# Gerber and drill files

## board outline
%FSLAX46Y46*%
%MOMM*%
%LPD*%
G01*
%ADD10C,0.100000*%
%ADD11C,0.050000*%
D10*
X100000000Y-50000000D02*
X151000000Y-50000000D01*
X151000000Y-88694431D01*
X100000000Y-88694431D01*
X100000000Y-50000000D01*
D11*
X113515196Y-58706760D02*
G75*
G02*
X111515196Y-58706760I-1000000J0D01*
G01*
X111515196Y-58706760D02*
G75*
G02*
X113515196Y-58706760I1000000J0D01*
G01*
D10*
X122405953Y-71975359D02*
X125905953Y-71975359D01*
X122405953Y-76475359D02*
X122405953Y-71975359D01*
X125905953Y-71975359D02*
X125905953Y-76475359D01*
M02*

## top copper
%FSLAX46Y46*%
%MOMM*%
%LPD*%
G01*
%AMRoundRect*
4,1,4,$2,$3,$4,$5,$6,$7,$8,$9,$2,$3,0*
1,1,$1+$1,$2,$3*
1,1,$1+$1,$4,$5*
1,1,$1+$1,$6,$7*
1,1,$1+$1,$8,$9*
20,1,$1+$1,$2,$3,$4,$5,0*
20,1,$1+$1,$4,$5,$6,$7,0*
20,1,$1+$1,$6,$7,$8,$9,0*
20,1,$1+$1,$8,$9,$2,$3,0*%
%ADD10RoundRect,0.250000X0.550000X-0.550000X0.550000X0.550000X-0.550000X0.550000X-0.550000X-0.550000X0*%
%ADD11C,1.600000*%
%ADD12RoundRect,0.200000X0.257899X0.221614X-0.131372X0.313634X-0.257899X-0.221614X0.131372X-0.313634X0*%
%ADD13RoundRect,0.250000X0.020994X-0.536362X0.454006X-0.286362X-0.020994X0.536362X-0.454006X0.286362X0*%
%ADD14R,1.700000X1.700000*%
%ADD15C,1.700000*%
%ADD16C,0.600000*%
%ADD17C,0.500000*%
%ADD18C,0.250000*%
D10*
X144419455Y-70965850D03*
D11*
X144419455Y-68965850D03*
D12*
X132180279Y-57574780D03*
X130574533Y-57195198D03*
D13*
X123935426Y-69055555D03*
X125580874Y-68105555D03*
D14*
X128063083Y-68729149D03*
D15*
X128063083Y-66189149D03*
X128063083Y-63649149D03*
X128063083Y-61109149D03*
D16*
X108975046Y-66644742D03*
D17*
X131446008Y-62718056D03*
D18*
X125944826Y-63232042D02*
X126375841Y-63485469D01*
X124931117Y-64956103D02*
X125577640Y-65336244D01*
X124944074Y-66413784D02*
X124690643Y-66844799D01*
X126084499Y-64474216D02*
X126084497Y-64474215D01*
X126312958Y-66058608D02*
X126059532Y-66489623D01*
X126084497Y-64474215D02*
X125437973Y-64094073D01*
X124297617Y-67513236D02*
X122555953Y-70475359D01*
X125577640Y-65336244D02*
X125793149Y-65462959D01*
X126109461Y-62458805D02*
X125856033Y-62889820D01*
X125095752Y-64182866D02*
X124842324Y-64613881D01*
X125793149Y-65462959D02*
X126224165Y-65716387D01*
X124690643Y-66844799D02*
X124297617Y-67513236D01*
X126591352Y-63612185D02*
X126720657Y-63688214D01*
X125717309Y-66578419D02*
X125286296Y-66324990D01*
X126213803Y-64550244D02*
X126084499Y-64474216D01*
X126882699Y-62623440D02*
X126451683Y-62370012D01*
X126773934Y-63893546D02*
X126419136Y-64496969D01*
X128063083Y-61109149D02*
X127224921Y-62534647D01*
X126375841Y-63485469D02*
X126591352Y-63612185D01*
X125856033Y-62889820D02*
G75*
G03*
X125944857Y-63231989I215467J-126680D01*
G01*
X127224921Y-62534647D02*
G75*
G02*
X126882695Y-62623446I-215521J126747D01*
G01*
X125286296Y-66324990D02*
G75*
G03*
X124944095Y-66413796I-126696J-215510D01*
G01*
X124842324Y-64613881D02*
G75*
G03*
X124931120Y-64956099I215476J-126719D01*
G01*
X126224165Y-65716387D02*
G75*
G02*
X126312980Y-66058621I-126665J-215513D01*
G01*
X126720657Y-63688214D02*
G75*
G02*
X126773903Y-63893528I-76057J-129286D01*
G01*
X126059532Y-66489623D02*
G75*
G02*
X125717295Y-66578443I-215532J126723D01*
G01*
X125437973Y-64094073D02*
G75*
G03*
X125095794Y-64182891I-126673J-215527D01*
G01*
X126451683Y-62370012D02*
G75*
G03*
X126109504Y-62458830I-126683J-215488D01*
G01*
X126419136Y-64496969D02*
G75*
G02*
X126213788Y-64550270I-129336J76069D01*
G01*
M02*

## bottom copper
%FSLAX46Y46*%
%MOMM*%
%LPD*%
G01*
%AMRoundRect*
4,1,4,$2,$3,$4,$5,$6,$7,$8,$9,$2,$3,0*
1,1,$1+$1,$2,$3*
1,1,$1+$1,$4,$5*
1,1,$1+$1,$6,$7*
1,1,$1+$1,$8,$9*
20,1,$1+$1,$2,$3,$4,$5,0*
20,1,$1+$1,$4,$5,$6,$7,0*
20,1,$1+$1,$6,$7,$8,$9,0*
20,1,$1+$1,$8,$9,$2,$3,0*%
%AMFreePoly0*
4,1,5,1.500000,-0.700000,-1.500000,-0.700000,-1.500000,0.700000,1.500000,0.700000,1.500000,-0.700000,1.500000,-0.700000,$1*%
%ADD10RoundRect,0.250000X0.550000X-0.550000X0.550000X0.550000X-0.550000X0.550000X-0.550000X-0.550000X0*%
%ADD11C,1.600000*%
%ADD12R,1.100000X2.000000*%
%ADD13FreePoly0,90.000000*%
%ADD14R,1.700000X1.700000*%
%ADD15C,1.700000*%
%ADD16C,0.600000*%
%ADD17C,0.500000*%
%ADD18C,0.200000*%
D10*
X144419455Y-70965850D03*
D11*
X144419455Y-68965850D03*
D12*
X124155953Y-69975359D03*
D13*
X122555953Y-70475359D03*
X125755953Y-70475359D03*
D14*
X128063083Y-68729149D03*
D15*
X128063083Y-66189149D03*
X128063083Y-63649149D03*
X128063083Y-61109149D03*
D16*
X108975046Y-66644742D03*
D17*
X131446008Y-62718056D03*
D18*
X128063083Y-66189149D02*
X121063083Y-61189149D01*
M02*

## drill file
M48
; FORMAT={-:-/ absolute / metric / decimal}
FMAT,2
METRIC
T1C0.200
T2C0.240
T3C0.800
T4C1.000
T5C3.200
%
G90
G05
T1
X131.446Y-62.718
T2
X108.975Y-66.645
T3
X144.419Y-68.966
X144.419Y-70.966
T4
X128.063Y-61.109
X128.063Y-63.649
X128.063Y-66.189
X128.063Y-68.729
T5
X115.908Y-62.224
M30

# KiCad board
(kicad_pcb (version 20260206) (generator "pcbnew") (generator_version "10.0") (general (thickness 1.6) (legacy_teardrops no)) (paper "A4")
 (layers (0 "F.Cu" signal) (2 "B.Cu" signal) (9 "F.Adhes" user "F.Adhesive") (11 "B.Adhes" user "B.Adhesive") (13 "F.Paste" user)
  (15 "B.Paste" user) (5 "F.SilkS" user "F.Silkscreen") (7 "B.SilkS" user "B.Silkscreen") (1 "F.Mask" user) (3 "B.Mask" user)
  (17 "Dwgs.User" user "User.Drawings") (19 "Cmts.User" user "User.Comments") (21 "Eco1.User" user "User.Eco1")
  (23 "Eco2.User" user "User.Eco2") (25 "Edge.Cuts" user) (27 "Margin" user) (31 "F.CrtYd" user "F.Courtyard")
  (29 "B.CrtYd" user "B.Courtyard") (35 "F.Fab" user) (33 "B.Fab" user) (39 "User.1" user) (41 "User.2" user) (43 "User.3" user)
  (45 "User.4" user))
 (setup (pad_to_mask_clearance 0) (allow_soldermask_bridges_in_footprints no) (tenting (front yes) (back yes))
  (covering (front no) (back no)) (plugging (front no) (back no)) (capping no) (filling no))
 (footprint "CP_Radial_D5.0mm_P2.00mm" (layer "F.Cu") (at 144.419455 70.96585 90)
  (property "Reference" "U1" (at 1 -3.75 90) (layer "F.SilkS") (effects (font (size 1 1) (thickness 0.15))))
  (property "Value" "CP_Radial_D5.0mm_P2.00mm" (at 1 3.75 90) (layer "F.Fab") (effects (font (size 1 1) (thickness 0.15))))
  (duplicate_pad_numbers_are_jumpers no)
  (pad "1" thru_hole roundrect (at 0 0 90) (size 1.6 1.6) (drill 0.8) (layers "*.Cu" "*.Mask") (remove_unused_layers no)
   (roundrect_rratio 0.15625) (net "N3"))
  (pad "2" thru_hole circle (at 2 0 90) (size 1.6 1.6) (drill 0.8) (layers "*.Cu" "*.Mask") (remove_unused_layers no) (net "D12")))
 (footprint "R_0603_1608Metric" (layer "F.Cu") (at 131.377406 57.384989 166.7)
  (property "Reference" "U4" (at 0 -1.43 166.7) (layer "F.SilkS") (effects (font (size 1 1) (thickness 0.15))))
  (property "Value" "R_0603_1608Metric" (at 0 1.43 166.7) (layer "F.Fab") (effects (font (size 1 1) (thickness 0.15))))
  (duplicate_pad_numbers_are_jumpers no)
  (pad "1" smd roundrect (at -0.825 0 166.7) (size 0.8 0.95) (layers "F.Cu" "F.Mask" "F.Paste") (roundrect_rratio 0.25) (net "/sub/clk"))
  (pad "2" smd roundrect (at 0.825 0 166.7) (size 0.8 0.95) (layers "F.Cu" "F.Mask" "F.Paste") (roundrect_rratio 0.25) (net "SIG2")))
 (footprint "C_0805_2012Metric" (layer "F.Cu") (at 124.75815 68.580555 30)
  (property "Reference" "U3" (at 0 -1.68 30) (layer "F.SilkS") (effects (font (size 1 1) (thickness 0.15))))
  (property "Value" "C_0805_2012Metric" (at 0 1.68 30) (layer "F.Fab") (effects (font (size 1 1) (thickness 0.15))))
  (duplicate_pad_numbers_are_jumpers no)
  (pad "1" smd roundrect (at -0.95 0 30) (size 1 1.45) (layers "F.Cu" "F.Mask" "F.Paste") (roundrect_rratio 0.25) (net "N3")
   (clearance 0.35))
  (pad "2" smd roundrect (at 0.95 0 30) (size 1 1.45) (layers "F.Cu" "F.Mask" "F.Paste") (roundrect_rratio 0.25)))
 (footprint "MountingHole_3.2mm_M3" (layer "F.Cu") (at 115.908484 62.224067 45)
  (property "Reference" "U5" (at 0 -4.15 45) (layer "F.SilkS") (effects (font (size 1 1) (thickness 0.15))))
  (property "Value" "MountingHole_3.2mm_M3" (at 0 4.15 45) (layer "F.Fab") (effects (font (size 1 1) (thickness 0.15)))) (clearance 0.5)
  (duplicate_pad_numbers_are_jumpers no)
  (pad "" np_thru_hole circle (at 0 0 45) (size 3.2 3.2) (drill 3.2) (layers "*.Cu" "*.Mask")))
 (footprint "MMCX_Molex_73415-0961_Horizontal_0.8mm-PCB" (layer "B.Cu") (at 124.155953 72.725359 90)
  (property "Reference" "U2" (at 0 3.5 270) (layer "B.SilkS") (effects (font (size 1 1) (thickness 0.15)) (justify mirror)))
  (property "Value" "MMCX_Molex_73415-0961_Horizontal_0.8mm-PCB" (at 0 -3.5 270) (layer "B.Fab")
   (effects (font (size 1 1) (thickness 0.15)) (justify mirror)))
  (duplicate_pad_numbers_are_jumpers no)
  (fp_line (start 0.75 -1.75) (end 0.75 1.75) (stroke (width 0.1) (type solid)) (layer "Edge.Cuts"))
  (fp_line (start -3.75 -1.75) (end 0.75 -1.75) (stroke (width 0.1) (type solid)) (layer "Edge.Cuts"))
  (fp_line (start 0.75 1.75) (end -3.75 1.75) (stroke (width 0.1) (type solid)) (layer "Edge.Cuts"))
  (pad "1" smd rect (at 2.75 0 90) (size 2 1.1) (layers "B.Cu" "B.Mask" "B.Paste") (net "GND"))
  (pad "2" smd custom (at 2.25 -1.6 90) (size 3 1.4) (layers "B.Cu" "B.Mask" "B.Paste") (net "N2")
   (options (clearance outline) (anchor rect)) (primitives))
  (pad "2" smd custom (at 2.25 1.6 90) (size 3 1.4) (layers "B.Cu" "B.Mask" "B.Paste") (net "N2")
   (options (clearance outline) (anchor rect)) (primitives)))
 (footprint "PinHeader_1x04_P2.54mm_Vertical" (layer "B.Cu") (at 128.063083 68.729149)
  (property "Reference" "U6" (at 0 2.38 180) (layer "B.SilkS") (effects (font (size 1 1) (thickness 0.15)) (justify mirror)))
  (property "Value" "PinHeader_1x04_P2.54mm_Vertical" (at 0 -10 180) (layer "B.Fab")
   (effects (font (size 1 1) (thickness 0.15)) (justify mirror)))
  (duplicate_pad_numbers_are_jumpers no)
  (pad "1" thru_hole rect (at 0 0) (size 1.7 1.7) (drill 1) (layers "*.Cu" "*.Mask") (remove_unused_layers no) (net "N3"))
  (pad "2" thru_hole circle (at 0 -2.54) (size 1.7 1.7) (drill 1) (layers "*.Cu" "*.Mask") (remove_unused_layers no) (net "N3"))
  (pad "3" thru_hole circle (at 0 -5.08) (size 1.7 1.7) (drill 1) (layers "*.Cu" "*.Mask") (remove_unused_layers no) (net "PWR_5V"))
  (pad "4" thru_hole circle (at 0 -7.62) (size 1.7 1.7) (drill 1) (layers "*.Cu" "*.Mask") (remove_unused_layers no)))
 (gr_rect (start 100 50) (end 151 88.694431) (stroke (width 0.1) (type default)) (fill no) (layer "Edge.Cuts"))
 (gr_circle (center 112.515196 58.70676) (end 113.515196 58.70676) (stroke (width 0.05) (type default)) (fill no) (layer "Edge.Cuts"))
 (segment (start 125.944826 63.232042) (end 126.375841 63.485469) (width 0.25) (layer "F.Cu") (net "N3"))
 (segment (start 124.931117 64.956103) (end 125.57764 65.336244) (width 0.25) (layer "F.Cu") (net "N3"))
 (segment (start 124.944074 66.413784) (end 124.690643 66.844799) (width 0.25) (layer "F.Cu") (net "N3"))
 (segment (start 126.084499 64.474216) (end 126.084497 64.474215) (width 0.25) (layer "F.Cu") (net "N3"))
 (segment (start 126.312958 66.058608) (end 126.059532 66.489623) (width 0.25) (layer "F.Cu") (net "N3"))
 (segment (start 126.084497 64.474215) (end 125.437973 64.094073) (width 0.25) (layer "F.Cu") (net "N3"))
 (segment (start 124.297617 67.513236) (end 122.555953 70.475359) (width 0.25) (layer "F.Cu") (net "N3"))
 (segment (start 125.57764 65.336244) (end 125.793149 65.462959) (width 0.25) (layer "F.Cu") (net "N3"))
 (segment (start 126.109461 62.458805) (end 125.856033 62.88982) (width 0.25) (layer "F.Cu") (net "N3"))
 (segment (start 125.095752 64.182866) (end 124.842324 64.613881) (width 0.25) (layer "F.Cu") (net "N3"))
 (segment (start 125.793149 65.462959) (end 126.224165 65.716387) (width 0.25) (layer "F.Cu") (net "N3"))
 (segment (start 124.690643 66.844799) (end 124.297617 67.513236) (width 0.25) (layer "F.Cu") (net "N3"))
 (segment (start 126.591352 63.612185) (end 126.720657 63.688214) (width 0.25) (layer "F.Cu") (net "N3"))
 (segment (start 125.717309 66.578419) (end 125.286296 66.32499) (width 0.25) (layer "F.Cu") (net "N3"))
 (segment (start 126.213803 64.550244) (end 126.084499 64.474216) (width 0.25) (layer "F.Cu") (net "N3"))
 (segment (start 126.882699 62.62344) (end 126.451683 62.370012) (width 0.25) (layer "F.Cu") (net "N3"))
 (segment (start 126.773934 63.893546) (end 126.419136 64.496969) (width 0.25) (layer "F.Cu") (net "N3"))
 (segment (start 128.063083 61.109149) (end 127.224921 62.534647) (width 0.25) (layer "F.Cu") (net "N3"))
 (segment (start 126.375841 63.485469) (end 126.591352 63.612185) (width 0.25) (layer "F.Cu") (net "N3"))
 (arc (start 125.856033 62.88982) (mid 125.829553 63.07932) (end 125.944826 63.232042) (width 0.25) (layer "F.Cu") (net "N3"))
 (arc (start 127.224921 62.534647) (mid 127.072199 62.64992) (end 126.882699 62.62344) (width 0.25) (layer "F.Cu") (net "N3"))
 (arc (start 125.286296 66.32499) (mid 125.096795 66.298511) (end 124.944074 66.413784) (width 0.25) (layer "F.Cu") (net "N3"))
 (arc (start 124.842324 64.613881) (mid 124.815844 64.803381) (end 124.931117 64.956103) (width 0.25) (layer "F.Cu") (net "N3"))
 (arc (start 126.224165 65.716387) (mid 126.339439 65.869107) (end 126.312958 66.058608) (width 0.25) (layer "F.Cu") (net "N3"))
 (arc (start 126.720657 63.688214) (mid 126.789821 63.779846) (end 126.773934 63.893546) (width 0.25) (layer "F.Cu") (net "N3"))
 (arc (start 126.059532 66.489623) (mid 125.906812 66.604897) (end 125.717309 66.578419) (width 0.25) (layer "F.Cu") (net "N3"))
 (arc (start 125.437973 64.094073) (mid 125.248473 64.067593) (end 125.095752 64.182866) (width 0.25) (layer "F.Cu") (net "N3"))
 (arc (start 126.451683 62.370012) (mid 126.262183 62.343532) (end 126.109461 62.458805) (width 0.25) (layer "F.Cu") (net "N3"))
 (arc (start 126.419136 64.496969) (mid 126.327503 64.566132) (end 126.213803 64.550244) (width 0.25) (layer "F.Cu") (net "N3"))
 (segment (start 128.063083 66.189149) (end 121.063083 61.189149) (width 0.2) (layer "B.Cu") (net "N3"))
 (via (at 108.975046 66.644742) (size 0.6) (drill 0.24) (layers "F.Cu" "B.Cu") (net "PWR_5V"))
 (via (at 131.446008 62.718056) (size 0.5) (drill 0.2) (layers "F.Cu" "B.Cu") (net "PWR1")))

